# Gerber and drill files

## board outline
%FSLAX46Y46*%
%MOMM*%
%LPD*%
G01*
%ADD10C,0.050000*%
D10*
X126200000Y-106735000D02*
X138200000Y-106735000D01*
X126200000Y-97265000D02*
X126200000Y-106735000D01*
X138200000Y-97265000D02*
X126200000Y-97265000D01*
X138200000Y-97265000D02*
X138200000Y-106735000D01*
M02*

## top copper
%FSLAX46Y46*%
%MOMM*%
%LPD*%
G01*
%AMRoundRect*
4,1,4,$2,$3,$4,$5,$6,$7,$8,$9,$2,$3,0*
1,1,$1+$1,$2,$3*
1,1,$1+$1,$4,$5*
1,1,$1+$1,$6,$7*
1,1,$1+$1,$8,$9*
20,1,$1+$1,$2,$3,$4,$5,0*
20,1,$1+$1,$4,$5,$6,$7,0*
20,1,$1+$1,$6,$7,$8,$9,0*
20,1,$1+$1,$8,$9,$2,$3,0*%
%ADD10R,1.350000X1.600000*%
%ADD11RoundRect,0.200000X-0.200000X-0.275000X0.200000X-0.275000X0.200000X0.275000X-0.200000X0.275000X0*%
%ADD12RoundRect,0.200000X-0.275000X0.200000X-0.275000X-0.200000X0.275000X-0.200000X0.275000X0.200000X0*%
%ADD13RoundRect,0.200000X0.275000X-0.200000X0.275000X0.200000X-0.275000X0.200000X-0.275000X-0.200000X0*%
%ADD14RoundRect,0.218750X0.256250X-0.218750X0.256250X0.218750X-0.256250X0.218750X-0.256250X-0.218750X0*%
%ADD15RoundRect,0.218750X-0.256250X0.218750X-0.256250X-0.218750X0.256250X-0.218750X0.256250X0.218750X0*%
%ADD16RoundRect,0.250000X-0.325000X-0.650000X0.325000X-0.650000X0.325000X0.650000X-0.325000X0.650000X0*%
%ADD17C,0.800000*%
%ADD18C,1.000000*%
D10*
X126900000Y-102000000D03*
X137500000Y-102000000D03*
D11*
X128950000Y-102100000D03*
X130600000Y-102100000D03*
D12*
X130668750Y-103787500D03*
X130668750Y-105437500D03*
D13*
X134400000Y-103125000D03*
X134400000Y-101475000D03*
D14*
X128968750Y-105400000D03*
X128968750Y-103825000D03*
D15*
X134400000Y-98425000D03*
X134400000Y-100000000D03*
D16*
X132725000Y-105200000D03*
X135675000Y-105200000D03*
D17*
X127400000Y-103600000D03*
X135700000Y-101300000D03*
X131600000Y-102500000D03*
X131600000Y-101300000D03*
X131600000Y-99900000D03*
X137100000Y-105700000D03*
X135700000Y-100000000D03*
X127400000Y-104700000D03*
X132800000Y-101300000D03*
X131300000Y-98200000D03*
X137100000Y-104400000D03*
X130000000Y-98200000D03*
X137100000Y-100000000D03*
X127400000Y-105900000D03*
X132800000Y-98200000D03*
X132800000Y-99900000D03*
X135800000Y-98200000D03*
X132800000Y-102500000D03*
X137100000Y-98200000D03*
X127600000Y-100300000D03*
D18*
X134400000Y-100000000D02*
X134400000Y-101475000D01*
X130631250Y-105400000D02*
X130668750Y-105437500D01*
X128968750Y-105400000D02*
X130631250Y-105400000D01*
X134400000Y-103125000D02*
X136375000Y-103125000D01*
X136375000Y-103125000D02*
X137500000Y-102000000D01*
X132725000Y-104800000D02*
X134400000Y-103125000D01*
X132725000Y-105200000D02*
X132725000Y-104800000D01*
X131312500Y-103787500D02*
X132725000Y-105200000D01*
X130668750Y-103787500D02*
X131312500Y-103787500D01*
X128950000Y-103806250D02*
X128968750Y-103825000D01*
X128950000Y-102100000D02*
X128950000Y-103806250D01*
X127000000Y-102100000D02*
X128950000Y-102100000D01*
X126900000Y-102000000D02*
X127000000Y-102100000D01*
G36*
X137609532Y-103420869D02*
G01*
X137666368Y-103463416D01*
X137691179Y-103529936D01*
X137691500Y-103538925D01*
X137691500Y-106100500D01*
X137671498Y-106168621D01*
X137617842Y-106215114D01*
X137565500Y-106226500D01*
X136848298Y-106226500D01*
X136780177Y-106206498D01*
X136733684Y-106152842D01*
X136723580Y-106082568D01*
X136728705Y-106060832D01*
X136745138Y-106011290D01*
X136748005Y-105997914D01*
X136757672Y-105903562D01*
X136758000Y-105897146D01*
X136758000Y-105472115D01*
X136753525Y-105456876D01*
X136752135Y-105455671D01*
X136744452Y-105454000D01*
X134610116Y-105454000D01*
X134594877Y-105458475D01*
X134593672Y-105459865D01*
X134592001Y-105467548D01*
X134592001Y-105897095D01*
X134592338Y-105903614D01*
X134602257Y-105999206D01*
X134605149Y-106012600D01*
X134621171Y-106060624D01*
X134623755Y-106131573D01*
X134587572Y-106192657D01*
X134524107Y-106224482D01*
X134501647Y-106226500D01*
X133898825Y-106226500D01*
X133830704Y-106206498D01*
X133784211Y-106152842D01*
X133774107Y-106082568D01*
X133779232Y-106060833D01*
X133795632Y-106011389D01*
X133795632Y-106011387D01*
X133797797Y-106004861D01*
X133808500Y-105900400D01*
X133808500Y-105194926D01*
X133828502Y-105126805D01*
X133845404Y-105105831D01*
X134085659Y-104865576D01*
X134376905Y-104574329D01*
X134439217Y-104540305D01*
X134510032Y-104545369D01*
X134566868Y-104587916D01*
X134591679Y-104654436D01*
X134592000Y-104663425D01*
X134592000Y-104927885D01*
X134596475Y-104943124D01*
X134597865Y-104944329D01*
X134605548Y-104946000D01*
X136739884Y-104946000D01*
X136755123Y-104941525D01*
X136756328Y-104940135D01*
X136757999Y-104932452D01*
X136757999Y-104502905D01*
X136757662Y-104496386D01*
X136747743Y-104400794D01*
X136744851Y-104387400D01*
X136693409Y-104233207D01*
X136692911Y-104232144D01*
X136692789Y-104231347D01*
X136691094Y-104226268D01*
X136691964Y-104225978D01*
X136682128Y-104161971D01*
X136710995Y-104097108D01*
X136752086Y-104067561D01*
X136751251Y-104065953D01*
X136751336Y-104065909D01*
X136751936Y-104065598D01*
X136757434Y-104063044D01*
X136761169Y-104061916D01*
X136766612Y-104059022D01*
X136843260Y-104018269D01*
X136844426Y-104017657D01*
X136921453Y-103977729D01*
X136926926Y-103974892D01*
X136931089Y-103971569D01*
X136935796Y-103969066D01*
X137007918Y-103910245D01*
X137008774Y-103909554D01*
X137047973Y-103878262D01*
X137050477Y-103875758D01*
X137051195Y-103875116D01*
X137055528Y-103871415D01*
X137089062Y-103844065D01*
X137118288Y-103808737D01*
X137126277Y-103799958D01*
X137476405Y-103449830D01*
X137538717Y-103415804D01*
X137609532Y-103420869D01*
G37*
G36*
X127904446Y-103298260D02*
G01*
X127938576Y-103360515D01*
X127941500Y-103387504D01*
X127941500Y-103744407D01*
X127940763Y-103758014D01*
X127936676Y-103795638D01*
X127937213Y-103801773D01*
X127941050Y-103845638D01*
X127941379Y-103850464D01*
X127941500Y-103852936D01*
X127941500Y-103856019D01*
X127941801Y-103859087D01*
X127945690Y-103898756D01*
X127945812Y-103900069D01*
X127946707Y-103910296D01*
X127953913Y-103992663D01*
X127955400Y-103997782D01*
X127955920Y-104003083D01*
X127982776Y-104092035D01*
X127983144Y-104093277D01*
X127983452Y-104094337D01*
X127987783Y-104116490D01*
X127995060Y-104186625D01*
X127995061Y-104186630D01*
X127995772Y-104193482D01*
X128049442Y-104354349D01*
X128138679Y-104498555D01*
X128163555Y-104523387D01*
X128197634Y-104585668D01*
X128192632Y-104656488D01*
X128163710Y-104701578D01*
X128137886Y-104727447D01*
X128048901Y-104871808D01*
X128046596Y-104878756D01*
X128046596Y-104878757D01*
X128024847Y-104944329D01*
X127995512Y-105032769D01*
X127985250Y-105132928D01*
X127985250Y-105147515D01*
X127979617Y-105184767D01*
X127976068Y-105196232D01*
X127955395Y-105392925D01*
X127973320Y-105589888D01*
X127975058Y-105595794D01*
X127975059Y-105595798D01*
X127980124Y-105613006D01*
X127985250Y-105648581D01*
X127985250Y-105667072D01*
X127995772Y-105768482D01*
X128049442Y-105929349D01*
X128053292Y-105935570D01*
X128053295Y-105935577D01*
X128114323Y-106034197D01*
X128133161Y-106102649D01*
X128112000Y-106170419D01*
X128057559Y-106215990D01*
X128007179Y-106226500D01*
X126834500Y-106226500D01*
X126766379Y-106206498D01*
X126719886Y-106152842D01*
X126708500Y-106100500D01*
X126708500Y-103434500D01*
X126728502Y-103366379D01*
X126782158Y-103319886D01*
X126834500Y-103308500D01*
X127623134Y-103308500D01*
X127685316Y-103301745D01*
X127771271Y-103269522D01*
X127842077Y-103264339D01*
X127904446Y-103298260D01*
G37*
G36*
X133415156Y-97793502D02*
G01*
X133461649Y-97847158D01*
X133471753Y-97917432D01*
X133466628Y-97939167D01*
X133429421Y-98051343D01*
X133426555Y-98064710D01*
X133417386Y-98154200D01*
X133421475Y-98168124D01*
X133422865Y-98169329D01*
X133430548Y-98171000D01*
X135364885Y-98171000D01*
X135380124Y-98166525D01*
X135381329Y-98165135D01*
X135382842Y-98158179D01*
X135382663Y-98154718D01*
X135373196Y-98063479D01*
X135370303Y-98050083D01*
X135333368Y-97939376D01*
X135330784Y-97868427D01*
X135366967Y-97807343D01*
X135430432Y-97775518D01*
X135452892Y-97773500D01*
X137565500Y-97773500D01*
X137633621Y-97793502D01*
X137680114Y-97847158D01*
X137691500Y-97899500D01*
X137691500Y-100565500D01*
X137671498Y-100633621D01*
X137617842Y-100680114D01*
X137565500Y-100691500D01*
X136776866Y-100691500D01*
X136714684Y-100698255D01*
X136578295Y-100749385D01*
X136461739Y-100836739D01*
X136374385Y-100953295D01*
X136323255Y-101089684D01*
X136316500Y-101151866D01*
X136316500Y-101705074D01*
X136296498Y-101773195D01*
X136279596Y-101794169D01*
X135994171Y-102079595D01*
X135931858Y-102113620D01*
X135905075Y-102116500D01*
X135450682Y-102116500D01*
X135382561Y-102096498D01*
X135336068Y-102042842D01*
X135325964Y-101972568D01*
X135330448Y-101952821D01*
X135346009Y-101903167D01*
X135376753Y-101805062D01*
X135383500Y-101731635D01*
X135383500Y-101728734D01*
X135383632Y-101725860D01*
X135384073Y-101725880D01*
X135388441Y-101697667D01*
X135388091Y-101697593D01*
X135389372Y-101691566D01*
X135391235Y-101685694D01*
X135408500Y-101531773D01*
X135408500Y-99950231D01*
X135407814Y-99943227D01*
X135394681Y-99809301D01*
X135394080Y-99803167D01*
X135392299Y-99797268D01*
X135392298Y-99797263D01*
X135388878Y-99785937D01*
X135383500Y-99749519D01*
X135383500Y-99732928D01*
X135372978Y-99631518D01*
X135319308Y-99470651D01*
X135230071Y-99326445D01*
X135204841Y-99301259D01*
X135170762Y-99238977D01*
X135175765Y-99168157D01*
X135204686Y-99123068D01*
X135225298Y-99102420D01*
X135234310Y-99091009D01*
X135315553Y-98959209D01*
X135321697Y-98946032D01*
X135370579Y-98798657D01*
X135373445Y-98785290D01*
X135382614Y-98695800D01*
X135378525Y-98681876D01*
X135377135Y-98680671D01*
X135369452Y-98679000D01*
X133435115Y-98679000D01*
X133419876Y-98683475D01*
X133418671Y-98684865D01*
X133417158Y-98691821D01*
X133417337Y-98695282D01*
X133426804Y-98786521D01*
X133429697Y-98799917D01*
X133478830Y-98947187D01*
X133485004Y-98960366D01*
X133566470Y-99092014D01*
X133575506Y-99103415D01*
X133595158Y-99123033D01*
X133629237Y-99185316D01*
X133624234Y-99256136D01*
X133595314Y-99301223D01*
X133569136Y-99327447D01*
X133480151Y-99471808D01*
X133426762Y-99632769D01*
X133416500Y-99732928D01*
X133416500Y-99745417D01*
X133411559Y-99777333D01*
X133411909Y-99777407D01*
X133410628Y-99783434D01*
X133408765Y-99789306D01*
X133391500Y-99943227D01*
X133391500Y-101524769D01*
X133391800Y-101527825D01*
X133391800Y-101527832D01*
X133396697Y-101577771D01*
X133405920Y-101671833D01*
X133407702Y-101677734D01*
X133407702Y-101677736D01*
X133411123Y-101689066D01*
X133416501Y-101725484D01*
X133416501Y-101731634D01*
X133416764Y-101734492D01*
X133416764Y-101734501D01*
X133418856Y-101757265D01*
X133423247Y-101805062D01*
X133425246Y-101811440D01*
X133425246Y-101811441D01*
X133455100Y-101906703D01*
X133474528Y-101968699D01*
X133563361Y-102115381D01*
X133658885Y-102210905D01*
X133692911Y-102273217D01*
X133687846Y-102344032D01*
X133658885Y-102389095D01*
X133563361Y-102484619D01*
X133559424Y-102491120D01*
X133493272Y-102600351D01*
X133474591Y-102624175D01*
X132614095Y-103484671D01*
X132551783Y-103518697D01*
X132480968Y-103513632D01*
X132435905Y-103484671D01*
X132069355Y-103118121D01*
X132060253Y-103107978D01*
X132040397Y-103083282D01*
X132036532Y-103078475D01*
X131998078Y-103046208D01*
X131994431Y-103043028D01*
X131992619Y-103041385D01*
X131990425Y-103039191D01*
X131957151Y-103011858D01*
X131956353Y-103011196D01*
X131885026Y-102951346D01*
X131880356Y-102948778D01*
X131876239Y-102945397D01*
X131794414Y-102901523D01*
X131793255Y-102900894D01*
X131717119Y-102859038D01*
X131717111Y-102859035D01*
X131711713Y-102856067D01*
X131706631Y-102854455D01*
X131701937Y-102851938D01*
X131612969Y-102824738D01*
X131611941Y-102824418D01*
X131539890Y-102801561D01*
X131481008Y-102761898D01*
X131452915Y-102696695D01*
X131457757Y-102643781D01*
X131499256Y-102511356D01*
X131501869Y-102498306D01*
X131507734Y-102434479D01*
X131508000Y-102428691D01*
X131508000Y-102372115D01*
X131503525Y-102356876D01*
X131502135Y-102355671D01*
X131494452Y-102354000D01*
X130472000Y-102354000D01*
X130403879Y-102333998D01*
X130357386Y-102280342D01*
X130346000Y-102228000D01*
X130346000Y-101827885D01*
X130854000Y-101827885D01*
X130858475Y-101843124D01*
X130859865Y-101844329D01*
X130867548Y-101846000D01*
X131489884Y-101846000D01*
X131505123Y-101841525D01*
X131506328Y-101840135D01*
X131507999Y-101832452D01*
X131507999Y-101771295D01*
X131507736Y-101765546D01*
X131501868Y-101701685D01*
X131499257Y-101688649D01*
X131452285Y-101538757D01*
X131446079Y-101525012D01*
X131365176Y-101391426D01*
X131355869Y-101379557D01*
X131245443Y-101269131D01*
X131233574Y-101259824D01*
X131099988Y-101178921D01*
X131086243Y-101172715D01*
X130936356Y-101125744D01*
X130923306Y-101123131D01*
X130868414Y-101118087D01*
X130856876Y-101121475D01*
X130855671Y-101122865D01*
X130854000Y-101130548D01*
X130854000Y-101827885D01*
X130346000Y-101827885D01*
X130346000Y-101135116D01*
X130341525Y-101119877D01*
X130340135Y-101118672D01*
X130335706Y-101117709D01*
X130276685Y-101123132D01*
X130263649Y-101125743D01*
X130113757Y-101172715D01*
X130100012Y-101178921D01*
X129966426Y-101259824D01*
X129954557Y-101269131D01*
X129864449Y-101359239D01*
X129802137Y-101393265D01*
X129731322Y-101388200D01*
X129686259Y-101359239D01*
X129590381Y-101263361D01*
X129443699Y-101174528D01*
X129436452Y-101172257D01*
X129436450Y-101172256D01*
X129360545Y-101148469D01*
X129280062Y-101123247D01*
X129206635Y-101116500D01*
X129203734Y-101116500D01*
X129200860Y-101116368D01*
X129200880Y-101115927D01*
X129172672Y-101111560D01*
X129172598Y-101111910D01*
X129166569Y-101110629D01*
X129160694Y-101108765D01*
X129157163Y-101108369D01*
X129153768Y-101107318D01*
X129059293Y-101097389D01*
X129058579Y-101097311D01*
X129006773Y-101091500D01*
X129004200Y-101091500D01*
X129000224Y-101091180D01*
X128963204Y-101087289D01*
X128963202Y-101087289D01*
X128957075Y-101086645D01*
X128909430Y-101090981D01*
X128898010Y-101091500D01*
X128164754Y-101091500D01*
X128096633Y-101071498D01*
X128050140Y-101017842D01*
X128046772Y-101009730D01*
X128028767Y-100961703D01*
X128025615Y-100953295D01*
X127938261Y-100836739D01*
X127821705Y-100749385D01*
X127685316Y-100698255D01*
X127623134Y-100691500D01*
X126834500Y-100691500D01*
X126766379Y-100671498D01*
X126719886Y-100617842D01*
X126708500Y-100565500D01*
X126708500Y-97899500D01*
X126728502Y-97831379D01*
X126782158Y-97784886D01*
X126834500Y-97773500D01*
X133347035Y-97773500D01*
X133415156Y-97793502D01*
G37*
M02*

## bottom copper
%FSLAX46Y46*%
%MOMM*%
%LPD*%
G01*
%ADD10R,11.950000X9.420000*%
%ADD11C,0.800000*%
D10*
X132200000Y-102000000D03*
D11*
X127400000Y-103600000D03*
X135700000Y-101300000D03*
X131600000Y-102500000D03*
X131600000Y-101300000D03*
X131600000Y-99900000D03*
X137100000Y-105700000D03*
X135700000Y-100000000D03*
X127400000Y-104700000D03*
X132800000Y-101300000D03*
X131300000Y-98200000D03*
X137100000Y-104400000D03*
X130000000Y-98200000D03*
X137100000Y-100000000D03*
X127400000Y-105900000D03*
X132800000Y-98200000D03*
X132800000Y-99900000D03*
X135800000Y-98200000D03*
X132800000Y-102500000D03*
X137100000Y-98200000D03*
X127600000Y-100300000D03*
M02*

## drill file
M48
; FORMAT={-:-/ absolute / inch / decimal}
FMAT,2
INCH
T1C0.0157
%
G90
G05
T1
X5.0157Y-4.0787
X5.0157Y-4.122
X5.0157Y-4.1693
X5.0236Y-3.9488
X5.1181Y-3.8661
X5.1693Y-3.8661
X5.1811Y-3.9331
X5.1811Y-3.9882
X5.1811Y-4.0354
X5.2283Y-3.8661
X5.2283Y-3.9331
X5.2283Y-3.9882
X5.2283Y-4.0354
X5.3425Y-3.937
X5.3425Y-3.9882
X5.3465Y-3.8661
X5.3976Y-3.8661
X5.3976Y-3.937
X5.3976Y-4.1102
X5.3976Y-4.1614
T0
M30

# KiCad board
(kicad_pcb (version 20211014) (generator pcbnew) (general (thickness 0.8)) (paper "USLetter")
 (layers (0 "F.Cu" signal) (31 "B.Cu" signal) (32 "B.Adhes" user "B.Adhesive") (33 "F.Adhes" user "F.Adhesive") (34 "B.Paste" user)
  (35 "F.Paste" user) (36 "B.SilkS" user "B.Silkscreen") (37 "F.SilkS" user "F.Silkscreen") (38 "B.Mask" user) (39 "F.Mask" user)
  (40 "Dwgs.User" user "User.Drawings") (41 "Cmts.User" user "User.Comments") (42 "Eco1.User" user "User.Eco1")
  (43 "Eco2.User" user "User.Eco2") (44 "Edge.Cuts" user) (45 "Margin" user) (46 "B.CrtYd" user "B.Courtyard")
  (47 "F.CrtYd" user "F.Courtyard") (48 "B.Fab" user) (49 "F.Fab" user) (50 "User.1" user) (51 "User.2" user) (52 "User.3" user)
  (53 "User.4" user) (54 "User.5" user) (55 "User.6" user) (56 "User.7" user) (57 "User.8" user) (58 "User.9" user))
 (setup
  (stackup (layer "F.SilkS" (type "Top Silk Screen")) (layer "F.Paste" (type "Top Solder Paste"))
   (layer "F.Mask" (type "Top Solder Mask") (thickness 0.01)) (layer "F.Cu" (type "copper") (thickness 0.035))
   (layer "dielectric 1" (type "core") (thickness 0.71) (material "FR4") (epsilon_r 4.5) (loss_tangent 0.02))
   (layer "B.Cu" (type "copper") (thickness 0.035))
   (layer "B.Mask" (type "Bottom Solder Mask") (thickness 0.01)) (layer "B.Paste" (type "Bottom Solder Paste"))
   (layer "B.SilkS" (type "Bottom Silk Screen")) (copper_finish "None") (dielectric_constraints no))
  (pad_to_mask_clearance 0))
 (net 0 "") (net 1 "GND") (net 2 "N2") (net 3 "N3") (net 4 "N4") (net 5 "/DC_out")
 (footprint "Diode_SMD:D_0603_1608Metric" (layer "F.Cu") (at 134.4 99.2125 -90)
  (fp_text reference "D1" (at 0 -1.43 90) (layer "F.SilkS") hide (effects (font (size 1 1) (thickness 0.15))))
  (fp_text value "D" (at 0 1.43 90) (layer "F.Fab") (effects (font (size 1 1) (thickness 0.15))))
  (pad "1" smd roundrect (at -0.7875 0 270) (size 0.875 0.95) (layers "F.Cu" "F.Paste" "F.Mask") (roundrect_rratio 0.25) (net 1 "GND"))
  (pad "2" smd roundrect (at 0.7875 0 270) (size 0.875 0.95) (layers "F.Cu" "F.Paste" "F.Mask") (roundrect_rratio 0.25) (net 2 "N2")))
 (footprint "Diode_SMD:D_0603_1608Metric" (layer "F.Cu") (at 128.96875 104.6125 90)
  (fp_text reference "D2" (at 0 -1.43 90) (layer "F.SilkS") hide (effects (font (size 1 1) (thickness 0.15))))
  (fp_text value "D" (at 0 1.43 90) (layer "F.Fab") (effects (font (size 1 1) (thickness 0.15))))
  (pad "1" smd roundrect (at -0.7875 0 90) (size 0.875 0.95) (layers "F.Cu" "F.Paste" "F.Mask") (roundrect_rratio 0.25) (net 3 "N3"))
  (pad "2" smd roundrect (at 0.7875 0 90) (size 0.875 0.95) (layers "F.Cu" "F.Paste" "F.Mask") (roundrect_rratio 0.25) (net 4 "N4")))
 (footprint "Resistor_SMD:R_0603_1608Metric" (layer "F.Cu") (at 130.66875 104.6125 -90)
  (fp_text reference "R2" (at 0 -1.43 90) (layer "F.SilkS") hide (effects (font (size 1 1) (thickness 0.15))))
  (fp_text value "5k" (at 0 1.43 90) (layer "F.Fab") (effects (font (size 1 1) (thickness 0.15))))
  (pad "1" smd roundrect (at -0.825 0 270) (size 0.8 0.95) (layers "F.Cu" "F.Paste" "F.Mask") (roundrect_rratio 0.25) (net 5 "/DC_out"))
  (pad "2" smd roundrect (at 0.825 0 270) (size 0.8 0.95) (layers "F.Cu" "F.Paste" "F.Mask") (roundrect_rratio 0.25) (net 3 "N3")))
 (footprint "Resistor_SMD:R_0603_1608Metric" (layer "F.Cu") (at 134.4 102.3 90)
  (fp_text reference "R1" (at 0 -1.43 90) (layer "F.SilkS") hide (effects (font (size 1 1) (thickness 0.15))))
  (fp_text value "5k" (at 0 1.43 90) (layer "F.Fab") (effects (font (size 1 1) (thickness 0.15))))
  (pad "1" smd roundrect (at -0.825 0 90) (size 0.8 0.95) (layers "F.Cu" "F.Paste" "F.Mask") (roundrect_rratio 0.25) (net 5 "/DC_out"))
  (pad "2" smd roundrect (at 0.825 0 90) (size 0.8 0.95) (layers "F.Cu" "F.Paste" "F.Mask") (roundrect_rratio 0.25) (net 2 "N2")))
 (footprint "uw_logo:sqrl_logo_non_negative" (layer "F.Cu") (at 127.7 98.6)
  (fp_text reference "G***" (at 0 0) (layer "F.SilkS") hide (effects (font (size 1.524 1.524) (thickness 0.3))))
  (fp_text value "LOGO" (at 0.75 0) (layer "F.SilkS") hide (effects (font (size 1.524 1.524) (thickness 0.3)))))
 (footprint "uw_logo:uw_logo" (layer "F.Cu") (at 129.5 100.1)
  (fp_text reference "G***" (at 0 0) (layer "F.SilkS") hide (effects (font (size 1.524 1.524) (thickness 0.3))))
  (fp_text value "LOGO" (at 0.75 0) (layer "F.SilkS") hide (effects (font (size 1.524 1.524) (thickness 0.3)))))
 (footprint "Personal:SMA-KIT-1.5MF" (layer "F.Cu") (at 132.2 102)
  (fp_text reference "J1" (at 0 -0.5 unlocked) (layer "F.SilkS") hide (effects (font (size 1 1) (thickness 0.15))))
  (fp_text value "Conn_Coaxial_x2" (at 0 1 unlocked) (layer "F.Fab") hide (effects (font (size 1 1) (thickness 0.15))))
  (fp_line (start -6 4.735) (end 6 4.735) (layer "Edge.Cuts") (width 0.05))
  (fp_line (start -6 -4.735) (end -6 4.735) (layer "Edge.Cuts") (width 0.05))
  (fp_line (start 6 -4.735) (end -6 -4.735) (layer "Edge.Cuts") (width 0.05))
  (fp_line (start 6 -4.735) (end 6 4.735) (layer "Edge.Cuts") (width 0.05))
  (pad "1" smd rect (at -5.3 0) (size 1.35 1.6) (layers "F.Cu" "F.Paste" "F.Mask") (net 4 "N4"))
  (pad "2" smd rect (at 5.3 0) (size 1.35 1.6) (layers "F.Cu" "F.Paste" "F.Mask") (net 5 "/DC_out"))
  (pad "3" smd rect (at 0 0) (size 11.95 9.42) (layers "B.Cu" "B.Paste" "B.Mask") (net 1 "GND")))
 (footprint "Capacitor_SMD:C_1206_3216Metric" (layer "F.Cu") (at 134.2 105.2)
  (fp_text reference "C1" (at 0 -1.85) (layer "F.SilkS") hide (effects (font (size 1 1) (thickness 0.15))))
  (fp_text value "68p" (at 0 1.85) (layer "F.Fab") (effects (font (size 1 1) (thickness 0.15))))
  (pad "1" smd roundrect (at -1.475 0) (size 1.15 1.8) (layers "F.Cu" "F.Paste" "F.Mask") (roundrect_rratio 0.2173913043) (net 5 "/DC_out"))
  (pad "2" smd roundrect (at 1.475 0) (size 1.15 1.8) (layers "F.Cu" "F.Paste" "F.Mask") (roundrect_rratio 0.2173913043) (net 1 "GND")))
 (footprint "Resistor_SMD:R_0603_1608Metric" (layer "F.Cu") (at 129.775 102.1)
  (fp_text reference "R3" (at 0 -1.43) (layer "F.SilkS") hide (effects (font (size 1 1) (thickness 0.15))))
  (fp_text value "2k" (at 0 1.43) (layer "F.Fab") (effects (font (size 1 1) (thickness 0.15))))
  (pad "1" smd roundrect (at -0.825 0) (size 0.8 0.95) (layers "F.Cu" "F.Paste" "F.Mask") (roundrect_rratio 0.25) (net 4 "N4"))
  (pad "2" smd roundrect (at 0.825 0) (size 0.8 0.95) (layers "F.Cu" "F.Paste" "F.Mask") (roundrect_rratio 0.25) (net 1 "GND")))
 (segment (start 127 102.1) (end 128.95 102.1) (width 1) (layer "F.Cu") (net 4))
 (segment (start 126.9 102) (end 127 102.1) (width 1) (layer "F.Cu") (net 4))
 (segment (start 128.95 103.80625) (end 128.96875 103.825) (width 1) (layer "F.Cu") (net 4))
 (segment (start 128.95 102.1) (end 128.95 103.80625) (width 1) (layer "F.Cu") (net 4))
 (via (at 135.7 100) (size 0.8) (drill 0.4) (layers "F.Cu" "B.Cu") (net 1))
 (via (at 135.7 101.3) (size 0.8) (drill 0.4) (layers "F.Cu" "B.Cu") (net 1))
 (via (at 127.4 104.7) (size 0.8) (drill 0.4) (layers "F.Cu" "B.Cu") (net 1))
 (via (at 132.8 101.3) (size 0.8) (drill 0.4) (layers "F.Cu" "B.Cu") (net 1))
 (via (at 137.1 105.7) (size 0.8) (drill 0.4) (layers "F.Cu" "B.Cu") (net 1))
 (via (at 131.3 98.2) (size 0.8) (drill 0.4) (layers "F.Cu" "B.Cu") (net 1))
 (via (at 137.1 104.4) (size 0.8) (drill 0.4) (layers "F.Cu" "B.Cu") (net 1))
 (via (at 130 98.2) (size 0.8) (drill 0.4) (layers "F.Cu" "B.Cu") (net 1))
 (via (at 137.1 100) (size 0.8) (drill 0.4) (layers "F.Cu" "B.Cu") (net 1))
 (via (at 127.4 105.9) (size 0.8) (drill 0.4) (layers "F.Cu" "B.Cu") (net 1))
 (via (at 131.6 101.3) (size 0.8) (drill 0.4) (layers "F.Cu" "B.Cu") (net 1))
 (via (at 127.4 103.6) (size 0.8) (drill 0.4) (layers "F.Cu" "B.Cu") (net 1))
 (via (at 132.8 98.2) (size 0.8) (drill 0.4) (layers "F.Cu" "B.Cu") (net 1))
 (via (at 132.8 99.9) (size 0.8) (drill 0.4) (layers "F.Cu" "B.Cu") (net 1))
 (via (at 135.8 98.2) (size 0.8) (drill 0.4) (layers "F.Cu" "B.Cu") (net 1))
 (via (at 132.8 102.5) (size 0.8) (drill 0.4) (layers "F.Cu" "B.Cu") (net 1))
 (via (at 137.1 98.2) (size 0.8) (drill 0.4) (layers "F.Cu" "B.Cu") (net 1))
 (via (at 127.6 100.3) (size 0.8) (drill 0.4) (layers "F.Cu" "B.Cu") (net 1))
 (via (at 131.6 99.9) (size 0.8) (drill 0.4) (layers "F.Cu" "B.Cu") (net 1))
 (via (at 131.6 102.5) (size 0.8) (drill 0.4) (layers "F.Cu" "B.Cu") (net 1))
 (segment (start 134.4 103.125) (end 136.375 103.125) (width 1) (layer "F.Cu") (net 5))
 (segment (start 132.725 105.2) (end 132.725 104.8) (width 1) (layer "F.Cu") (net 5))
 (segment (start 136.375 103.125) (end 137.5 102) (width 1) (layer "F.Cu") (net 5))
 (segment (start 130.66875 103.7875) (end 131.3125 103.7875) (width 1) (layer "F.Cu") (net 5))
 (segment (start 132.725 104.8) (end 134.4 103.125) (width 1) (layer "F.Cu") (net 5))
 (segment (start 131.3125 103.7875) (end 132.725 105.2) (width 1) (layer "F.Cu") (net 5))
 (segment (start 134.4 100) (end 134.4 101.475) (width 1) (layer "F.Cu") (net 2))
 (segment (start 128.96875 105.4) (end 130.63125 105.4) (width 1) (layer "F.Cu") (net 3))
 (segment (start 130.63125 105.4) (end 130.66875 105.4375) (width 1) (layer "F.Cu") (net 3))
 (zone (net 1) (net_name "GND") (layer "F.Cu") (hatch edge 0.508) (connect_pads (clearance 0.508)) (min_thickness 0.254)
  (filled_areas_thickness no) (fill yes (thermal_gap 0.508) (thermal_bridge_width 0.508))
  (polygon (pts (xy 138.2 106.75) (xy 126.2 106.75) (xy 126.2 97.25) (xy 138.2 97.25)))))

